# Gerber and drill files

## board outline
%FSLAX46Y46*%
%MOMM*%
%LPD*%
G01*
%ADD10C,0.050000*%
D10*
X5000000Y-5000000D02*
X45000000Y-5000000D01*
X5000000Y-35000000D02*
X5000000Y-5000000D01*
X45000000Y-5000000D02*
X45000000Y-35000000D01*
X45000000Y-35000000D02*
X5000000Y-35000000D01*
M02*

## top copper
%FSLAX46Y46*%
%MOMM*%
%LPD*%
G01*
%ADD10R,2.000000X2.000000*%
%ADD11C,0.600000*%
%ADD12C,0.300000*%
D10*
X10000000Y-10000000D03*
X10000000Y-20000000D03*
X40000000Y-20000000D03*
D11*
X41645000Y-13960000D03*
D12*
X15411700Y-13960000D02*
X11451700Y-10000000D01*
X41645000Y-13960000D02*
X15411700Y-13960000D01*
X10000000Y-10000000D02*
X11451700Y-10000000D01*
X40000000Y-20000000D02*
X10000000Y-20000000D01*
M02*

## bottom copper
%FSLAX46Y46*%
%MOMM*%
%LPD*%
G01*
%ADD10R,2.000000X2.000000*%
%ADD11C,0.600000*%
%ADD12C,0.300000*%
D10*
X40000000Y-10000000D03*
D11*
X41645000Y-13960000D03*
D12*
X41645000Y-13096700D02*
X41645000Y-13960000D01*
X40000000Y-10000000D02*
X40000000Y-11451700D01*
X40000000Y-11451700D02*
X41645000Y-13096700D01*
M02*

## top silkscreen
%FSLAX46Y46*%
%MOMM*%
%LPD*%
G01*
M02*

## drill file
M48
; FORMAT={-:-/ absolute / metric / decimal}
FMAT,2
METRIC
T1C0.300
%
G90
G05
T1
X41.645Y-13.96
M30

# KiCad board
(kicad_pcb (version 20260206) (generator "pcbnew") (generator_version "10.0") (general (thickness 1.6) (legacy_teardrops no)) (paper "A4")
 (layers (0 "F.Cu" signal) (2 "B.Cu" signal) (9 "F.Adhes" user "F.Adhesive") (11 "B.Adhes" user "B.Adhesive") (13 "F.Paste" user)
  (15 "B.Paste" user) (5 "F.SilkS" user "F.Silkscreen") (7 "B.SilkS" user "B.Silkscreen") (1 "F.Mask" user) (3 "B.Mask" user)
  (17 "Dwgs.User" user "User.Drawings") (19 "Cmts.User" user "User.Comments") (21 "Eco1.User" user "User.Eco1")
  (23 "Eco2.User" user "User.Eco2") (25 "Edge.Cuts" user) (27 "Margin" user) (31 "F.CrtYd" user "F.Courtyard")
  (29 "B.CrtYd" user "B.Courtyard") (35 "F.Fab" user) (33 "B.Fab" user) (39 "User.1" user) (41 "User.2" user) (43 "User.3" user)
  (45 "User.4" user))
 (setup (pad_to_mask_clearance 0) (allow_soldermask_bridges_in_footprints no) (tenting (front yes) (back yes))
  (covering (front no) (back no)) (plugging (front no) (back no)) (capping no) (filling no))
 (gr_line (start 5 5) (end 45 5) (stroke (width 0.05) (type default)) (layer "Edge.Cuts"))
 (gr_line (start 5 35) (end 5 5) (stroke (width 0.05) (type default)) (layer "Edge.Cuts"))
 (gr_line (start 45 5) (end 45 35) (stroke (width 0.05) (type default)) (layer "Edge.Cuts"))
 (gr_line (start 45 35) (end 5 35) (stroke (width 0.05) (type default)) (layer "Edge.Cuts"))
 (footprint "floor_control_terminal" (layer "F.Cu") (at 10 10)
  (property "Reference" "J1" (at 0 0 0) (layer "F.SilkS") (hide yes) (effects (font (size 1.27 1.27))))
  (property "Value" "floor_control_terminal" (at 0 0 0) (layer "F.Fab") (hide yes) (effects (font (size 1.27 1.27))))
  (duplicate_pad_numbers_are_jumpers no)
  (pad "1" smd rect (at 0 0) (size 2 2) (layers "F.Cu" "F.Paste" "F.Mask") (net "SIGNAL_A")))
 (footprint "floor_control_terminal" (layer "B.Cu") (at 40 10)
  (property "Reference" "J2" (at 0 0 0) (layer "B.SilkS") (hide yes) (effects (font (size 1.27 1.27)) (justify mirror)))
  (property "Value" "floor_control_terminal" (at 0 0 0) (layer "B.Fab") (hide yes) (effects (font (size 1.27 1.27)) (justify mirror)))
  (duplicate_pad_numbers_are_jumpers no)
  (pad "1" smd rect (at 0 0) (size 2 2) (layers "B.Cu" "B.Paste" "B.Mask") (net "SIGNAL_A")))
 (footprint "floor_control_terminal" (layer "F.Cu") (at 10 20)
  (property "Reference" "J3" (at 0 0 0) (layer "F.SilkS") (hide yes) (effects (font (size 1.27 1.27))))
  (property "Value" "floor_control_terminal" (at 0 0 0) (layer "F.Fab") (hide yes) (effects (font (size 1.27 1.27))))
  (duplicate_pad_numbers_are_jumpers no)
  (pad "1" smd rect (at 0 0) (size 2 2) (layers "F.Cu" "F.Paste" "F.Mask") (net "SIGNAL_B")))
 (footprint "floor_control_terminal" (layer "F.Cu") (at 40 20)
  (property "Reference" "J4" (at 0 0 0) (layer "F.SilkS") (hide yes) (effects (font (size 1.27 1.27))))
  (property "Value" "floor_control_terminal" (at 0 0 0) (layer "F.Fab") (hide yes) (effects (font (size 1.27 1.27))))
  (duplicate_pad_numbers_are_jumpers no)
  (pad "1" smd rect (at 0 0) (size 2 2) (layers "F.Cu" "F.Paste" "F.Mask") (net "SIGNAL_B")))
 (segment (start 15.4117 13.96) (end 11.4517 10) (width 0.3) (layer "F.Cu") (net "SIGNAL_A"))
 (segment (start 41.645 13.96) (end 15.4117 13.96) (width 0.3) (layer "F.Cu") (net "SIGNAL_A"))
 (segment (start 10 10) (end 11.4517 10) (width 0.3) (layer "F.Cu") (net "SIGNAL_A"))
 (via (at 41.645 13.96) (size 0.6) (drill 0.3) (layers "F.Cu" "B.Cu") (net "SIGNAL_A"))
 (segment (start 41.645 13.0967) (end 41.645 13.96) (width 0.3) (layer "B.Cu") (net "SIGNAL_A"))
 (segment (start 40 10) (end 40 11.4517) (width 0.3) (layer "B.Cu") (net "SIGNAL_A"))
 (segment (start 40 11.4517) (end 41.645 13.0967) (width 0.3) (layer "B.Cu") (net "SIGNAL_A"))
 (segment (start 40 20) (end 10 20) (width 0.3) (layer "F.Cu") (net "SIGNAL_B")))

